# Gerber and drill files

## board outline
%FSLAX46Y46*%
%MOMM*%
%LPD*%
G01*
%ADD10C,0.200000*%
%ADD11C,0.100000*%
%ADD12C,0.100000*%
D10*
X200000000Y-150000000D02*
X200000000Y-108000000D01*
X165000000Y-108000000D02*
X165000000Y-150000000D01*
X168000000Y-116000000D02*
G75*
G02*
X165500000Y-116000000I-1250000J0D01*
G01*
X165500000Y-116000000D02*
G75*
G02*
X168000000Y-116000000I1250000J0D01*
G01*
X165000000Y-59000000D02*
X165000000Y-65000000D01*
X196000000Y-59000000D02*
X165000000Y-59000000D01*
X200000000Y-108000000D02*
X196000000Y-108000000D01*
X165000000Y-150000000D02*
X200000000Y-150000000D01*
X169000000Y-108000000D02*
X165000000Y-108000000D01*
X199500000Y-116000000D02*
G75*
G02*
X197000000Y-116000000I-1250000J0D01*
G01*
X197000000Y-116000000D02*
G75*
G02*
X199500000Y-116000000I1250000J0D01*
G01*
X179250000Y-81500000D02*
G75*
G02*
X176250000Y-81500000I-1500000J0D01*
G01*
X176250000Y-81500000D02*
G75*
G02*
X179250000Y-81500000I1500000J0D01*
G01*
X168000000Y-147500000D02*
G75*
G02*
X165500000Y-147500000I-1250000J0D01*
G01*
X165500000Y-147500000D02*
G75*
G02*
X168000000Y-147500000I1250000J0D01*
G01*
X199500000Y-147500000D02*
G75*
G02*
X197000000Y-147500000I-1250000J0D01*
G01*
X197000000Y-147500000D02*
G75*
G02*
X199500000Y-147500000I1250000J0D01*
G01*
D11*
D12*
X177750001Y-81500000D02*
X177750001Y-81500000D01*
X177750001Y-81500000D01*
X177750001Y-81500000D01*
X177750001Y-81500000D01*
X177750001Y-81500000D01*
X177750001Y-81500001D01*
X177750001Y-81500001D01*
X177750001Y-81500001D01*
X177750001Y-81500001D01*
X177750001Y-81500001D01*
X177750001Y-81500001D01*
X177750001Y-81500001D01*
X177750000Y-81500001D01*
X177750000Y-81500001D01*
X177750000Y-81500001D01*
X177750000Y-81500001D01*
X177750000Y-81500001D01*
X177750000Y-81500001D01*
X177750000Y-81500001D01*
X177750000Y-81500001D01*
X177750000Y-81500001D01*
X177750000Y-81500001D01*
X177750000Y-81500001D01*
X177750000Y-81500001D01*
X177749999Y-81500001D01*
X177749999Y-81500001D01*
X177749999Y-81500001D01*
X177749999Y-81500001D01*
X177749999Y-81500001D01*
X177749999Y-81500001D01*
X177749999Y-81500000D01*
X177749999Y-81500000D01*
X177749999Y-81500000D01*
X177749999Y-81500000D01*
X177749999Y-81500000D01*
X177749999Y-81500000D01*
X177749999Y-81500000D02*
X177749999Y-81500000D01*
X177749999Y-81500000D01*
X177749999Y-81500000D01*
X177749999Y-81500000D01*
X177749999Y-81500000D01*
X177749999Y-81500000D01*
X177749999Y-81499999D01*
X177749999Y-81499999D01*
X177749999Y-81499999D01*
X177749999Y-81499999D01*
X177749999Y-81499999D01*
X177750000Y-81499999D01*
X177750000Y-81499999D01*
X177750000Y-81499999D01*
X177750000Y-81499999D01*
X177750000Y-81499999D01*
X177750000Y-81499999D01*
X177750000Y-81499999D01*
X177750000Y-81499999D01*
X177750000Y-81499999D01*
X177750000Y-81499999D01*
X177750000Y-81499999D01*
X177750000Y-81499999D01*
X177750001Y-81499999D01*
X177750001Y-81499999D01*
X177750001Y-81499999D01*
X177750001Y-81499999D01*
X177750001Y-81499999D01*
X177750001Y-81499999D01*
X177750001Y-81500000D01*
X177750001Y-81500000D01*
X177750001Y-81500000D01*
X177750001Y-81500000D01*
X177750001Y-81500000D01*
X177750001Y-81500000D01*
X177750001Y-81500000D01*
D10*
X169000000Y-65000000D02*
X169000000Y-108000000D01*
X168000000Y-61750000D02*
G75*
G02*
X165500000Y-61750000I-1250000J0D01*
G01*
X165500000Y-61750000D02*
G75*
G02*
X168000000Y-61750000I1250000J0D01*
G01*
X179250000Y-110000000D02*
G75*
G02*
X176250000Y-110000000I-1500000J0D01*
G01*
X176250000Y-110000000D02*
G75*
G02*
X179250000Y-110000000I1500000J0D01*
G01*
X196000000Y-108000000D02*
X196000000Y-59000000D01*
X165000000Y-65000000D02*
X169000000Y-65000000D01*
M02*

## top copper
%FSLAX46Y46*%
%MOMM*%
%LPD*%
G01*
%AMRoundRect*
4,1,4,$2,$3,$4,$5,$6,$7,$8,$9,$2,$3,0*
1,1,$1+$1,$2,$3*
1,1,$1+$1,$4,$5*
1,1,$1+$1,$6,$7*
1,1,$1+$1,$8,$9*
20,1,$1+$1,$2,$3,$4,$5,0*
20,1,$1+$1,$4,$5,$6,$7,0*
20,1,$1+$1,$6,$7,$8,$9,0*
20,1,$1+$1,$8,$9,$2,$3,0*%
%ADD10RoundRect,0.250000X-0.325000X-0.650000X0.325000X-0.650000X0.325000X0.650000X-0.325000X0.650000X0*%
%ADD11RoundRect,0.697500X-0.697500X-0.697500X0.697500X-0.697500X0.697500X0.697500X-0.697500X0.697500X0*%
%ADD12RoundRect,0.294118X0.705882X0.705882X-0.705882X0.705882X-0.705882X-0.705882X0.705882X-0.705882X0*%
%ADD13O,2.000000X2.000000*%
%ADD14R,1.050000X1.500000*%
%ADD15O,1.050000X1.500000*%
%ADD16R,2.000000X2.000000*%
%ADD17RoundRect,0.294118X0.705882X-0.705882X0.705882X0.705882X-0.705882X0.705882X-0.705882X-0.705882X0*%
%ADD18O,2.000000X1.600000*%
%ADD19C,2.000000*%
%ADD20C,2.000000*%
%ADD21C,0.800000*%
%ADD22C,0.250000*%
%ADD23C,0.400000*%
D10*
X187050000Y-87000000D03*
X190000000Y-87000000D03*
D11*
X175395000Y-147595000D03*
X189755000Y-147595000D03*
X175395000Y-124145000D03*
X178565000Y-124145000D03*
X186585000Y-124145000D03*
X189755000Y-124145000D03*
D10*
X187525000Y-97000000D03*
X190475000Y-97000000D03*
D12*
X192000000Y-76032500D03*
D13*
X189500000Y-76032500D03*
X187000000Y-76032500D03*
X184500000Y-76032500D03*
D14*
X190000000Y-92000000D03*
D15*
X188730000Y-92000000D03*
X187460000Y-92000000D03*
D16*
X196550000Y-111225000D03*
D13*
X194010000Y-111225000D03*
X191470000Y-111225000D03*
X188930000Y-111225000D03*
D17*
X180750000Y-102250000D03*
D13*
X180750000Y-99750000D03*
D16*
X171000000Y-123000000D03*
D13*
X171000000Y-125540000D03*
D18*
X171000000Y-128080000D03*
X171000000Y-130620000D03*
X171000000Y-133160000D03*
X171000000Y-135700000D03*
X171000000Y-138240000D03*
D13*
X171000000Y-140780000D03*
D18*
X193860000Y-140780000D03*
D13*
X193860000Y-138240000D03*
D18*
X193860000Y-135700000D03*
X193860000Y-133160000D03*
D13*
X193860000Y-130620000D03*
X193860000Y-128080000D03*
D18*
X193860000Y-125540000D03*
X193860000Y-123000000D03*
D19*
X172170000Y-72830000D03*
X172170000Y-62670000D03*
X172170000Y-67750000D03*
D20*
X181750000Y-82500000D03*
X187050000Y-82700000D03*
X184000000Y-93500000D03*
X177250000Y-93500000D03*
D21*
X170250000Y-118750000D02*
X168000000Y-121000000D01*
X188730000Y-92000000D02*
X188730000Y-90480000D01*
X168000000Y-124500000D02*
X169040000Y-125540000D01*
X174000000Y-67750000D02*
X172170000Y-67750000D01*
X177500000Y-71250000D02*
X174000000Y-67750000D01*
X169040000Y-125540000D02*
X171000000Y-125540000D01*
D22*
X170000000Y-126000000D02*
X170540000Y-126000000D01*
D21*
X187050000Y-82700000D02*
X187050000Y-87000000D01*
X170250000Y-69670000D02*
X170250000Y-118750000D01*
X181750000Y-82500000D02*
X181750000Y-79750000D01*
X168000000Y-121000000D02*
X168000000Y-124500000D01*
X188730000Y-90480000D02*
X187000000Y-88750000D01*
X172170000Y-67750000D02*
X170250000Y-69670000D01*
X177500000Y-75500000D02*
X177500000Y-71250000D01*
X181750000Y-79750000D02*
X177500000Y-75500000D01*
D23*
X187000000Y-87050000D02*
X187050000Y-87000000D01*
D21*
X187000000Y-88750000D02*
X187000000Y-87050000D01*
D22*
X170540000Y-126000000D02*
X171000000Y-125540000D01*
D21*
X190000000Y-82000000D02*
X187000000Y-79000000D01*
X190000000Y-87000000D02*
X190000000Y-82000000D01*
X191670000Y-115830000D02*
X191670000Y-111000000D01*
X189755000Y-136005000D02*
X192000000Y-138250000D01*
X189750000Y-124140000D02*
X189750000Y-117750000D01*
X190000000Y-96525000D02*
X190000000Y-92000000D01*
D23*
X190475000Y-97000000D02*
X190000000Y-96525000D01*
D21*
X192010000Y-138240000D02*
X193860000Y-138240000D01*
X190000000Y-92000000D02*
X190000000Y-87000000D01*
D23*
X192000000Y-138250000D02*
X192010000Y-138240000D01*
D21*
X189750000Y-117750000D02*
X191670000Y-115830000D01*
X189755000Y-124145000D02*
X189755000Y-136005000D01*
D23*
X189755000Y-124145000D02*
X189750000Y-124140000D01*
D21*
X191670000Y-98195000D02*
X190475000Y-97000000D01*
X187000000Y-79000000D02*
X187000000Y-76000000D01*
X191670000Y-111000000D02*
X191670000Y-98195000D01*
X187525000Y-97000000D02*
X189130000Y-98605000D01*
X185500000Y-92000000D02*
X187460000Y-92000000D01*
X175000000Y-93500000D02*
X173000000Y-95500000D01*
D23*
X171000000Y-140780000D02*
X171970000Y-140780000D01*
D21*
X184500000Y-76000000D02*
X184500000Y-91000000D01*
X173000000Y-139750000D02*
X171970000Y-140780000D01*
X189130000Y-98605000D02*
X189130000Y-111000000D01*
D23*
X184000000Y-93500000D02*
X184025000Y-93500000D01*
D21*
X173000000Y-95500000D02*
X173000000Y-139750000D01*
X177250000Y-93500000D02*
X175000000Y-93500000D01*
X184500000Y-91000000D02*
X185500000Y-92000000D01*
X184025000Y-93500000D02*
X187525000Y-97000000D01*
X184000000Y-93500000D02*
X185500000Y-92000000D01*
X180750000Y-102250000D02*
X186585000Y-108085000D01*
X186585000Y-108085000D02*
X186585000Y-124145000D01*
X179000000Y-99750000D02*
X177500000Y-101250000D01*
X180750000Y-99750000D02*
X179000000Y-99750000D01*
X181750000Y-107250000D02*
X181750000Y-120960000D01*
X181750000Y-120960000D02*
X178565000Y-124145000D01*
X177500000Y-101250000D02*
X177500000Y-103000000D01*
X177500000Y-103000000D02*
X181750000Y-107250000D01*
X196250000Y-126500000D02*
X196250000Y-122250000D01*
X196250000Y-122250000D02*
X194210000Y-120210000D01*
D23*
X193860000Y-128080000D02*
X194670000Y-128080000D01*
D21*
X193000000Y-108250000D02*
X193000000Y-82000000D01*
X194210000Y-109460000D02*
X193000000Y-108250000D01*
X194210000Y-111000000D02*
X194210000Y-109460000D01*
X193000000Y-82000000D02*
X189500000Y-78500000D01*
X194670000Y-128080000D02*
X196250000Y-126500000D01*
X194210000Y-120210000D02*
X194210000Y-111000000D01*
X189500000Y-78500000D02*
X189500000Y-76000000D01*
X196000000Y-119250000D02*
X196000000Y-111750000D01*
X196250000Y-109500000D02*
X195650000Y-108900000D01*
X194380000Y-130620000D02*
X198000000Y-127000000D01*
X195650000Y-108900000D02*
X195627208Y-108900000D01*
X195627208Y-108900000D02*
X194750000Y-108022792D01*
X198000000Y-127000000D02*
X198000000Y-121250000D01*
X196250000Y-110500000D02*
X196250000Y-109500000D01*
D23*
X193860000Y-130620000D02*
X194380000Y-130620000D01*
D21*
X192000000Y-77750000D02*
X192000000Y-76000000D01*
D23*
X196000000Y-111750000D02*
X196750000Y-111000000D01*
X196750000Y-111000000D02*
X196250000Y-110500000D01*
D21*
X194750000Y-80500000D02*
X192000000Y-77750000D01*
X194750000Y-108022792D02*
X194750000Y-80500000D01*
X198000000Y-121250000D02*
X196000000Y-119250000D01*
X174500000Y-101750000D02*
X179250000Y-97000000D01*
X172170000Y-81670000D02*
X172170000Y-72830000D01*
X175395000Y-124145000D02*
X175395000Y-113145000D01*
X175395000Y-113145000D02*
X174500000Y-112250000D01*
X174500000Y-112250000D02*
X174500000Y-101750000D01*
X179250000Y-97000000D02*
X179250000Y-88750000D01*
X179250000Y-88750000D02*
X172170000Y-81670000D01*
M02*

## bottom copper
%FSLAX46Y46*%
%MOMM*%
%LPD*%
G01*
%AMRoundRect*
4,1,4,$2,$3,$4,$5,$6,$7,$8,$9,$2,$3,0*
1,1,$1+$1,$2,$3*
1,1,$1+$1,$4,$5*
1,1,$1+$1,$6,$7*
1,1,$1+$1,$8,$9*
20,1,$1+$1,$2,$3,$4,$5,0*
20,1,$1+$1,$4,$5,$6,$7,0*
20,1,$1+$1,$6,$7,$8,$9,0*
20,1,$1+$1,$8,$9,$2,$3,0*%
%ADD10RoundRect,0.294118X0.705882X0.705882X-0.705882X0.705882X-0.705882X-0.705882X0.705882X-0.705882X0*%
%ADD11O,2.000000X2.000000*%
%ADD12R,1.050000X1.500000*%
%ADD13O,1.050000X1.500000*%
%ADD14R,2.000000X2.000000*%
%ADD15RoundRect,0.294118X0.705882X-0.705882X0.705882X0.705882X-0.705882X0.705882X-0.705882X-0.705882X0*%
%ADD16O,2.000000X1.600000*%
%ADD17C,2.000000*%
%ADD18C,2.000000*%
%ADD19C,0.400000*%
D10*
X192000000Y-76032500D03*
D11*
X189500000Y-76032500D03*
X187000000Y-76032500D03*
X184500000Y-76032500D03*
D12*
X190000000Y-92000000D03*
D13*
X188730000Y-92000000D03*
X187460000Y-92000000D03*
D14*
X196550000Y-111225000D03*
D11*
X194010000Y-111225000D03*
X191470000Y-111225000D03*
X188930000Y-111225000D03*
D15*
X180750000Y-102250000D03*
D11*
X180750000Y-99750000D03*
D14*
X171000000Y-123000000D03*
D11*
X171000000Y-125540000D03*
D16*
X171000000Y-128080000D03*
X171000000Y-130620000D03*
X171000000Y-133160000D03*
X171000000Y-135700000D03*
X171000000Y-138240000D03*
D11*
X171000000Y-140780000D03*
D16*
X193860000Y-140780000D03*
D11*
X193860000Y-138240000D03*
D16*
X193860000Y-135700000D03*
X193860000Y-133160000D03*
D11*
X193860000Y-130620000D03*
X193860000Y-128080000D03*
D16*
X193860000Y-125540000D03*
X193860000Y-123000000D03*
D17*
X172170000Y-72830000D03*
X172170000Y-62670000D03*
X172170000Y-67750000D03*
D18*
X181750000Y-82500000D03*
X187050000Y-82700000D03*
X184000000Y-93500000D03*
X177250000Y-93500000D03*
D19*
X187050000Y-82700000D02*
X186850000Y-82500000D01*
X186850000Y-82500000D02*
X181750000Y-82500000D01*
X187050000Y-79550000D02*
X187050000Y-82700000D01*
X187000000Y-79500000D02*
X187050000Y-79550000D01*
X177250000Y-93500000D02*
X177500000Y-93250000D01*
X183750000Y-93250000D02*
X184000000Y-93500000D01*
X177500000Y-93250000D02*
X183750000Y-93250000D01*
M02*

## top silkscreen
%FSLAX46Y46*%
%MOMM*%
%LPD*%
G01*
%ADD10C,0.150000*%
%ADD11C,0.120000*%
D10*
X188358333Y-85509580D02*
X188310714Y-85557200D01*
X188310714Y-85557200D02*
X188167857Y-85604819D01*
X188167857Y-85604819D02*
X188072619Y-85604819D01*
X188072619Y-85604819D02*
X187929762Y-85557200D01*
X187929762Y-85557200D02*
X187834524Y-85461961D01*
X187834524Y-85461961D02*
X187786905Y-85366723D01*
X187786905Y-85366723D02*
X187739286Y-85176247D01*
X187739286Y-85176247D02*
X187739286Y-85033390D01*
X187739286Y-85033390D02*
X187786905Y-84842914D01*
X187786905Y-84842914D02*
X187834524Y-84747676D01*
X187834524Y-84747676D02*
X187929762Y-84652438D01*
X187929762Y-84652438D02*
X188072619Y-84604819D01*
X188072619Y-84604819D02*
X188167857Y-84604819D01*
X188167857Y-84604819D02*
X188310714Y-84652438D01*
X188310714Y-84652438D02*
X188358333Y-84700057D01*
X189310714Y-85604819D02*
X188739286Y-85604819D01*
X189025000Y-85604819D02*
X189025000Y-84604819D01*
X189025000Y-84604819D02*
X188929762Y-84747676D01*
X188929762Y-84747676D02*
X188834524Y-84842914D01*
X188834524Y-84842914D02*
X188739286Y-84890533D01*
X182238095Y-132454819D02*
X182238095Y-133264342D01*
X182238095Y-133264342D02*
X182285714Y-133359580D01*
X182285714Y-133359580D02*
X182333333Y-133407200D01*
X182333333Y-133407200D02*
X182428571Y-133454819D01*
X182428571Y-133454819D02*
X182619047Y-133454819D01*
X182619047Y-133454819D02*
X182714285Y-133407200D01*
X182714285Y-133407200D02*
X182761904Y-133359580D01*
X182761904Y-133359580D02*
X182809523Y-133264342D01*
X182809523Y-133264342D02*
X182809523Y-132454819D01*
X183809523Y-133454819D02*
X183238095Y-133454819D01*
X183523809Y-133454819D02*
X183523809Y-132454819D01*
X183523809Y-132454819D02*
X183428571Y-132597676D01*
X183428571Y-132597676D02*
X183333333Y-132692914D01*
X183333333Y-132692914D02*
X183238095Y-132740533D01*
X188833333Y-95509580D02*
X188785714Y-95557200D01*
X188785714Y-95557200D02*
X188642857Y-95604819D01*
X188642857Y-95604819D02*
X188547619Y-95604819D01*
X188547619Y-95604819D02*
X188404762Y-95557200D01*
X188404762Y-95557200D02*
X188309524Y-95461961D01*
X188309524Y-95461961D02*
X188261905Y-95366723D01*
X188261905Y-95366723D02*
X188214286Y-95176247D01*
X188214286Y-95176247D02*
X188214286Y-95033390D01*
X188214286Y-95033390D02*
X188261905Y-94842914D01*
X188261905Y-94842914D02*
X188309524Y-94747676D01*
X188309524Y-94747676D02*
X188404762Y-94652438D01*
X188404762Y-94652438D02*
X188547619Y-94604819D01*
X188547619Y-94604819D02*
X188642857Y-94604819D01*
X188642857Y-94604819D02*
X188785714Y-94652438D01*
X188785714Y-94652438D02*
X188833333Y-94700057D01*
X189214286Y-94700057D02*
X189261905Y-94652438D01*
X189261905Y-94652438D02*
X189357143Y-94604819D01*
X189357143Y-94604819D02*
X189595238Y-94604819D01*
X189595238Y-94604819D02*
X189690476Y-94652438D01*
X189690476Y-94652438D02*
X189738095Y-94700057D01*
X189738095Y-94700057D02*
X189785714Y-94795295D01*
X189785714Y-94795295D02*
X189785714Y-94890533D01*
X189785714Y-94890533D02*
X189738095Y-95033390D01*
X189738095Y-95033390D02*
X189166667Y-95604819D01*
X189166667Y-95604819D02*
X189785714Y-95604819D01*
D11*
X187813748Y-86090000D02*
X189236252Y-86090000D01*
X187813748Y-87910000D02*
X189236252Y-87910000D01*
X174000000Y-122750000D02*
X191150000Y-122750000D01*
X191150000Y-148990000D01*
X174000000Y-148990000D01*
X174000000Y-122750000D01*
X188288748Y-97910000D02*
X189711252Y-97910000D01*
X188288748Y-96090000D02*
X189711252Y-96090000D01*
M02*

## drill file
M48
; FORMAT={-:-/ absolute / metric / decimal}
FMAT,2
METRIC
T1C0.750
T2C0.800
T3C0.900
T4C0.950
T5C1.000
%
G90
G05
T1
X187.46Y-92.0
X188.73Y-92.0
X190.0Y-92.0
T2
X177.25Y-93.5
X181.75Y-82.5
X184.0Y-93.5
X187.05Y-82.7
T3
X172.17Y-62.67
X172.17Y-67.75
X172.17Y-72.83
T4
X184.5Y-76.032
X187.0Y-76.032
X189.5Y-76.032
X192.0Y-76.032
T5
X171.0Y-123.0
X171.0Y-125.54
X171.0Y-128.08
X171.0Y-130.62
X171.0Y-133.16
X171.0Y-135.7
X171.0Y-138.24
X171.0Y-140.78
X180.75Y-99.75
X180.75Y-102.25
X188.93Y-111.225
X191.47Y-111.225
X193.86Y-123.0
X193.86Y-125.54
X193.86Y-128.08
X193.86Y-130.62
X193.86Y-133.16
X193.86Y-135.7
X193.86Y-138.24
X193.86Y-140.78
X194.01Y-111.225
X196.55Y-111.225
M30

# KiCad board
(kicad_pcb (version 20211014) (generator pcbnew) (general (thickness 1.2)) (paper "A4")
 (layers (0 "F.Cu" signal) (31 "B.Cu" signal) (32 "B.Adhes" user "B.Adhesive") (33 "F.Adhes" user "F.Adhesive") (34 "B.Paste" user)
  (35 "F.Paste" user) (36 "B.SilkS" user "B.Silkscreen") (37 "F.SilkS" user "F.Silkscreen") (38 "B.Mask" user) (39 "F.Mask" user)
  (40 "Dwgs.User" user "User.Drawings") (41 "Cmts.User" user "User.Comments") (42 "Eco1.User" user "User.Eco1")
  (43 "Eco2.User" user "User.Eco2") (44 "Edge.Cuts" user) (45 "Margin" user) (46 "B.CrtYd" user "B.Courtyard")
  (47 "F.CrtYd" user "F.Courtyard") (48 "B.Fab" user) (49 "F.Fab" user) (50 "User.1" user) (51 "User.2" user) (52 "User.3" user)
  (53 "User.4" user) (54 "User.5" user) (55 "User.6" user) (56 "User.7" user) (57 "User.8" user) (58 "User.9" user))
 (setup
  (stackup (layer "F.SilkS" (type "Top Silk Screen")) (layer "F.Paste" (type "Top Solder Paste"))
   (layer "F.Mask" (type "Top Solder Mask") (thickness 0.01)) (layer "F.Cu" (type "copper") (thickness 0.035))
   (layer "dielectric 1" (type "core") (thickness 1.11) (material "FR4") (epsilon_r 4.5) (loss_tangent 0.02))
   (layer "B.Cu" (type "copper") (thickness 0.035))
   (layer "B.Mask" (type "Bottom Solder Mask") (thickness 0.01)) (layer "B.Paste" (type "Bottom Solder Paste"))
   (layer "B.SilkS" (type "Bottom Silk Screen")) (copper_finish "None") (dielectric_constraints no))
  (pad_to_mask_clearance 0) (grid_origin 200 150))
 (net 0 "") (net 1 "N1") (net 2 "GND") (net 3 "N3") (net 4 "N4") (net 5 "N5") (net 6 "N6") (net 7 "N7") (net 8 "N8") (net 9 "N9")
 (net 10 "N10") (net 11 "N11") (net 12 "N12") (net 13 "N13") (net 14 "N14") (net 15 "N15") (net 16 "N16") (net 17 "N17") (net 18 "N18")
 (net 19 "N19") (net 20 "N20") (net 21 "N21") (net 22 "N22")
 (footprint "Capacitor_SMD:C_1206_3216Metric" (layer "F.Cu") (at 188.525 87)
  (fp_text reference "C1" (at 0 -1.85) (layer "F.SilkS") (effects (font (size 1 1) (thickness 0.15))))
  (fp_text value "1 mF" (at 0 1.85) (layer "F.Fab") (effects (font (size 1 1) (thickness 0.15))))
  (fp_line (start -0.711252 -0.91) (end 0.711252 -0.91) (layer "F.SilkS") (width 0.12))
  (fp_line (start -0.711252 0.91) (end 0.711252 0.91) (layer "F.SilkS") (width 0.12))
  (pad "1" smd roundrect (at -1.475 0) (size 1.15 1.8) (layers "F.Cu" "F.Paste" "F.Mask") (roundrect_rratio 0.217391) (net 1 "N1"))
  (pad "2" smd roundrect (at 1.475 0) (size 1.15 1.8) (layers "F.Cu" "F.Paste" "F.Mask") (roundrect_rratio 0.217391) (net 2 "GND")))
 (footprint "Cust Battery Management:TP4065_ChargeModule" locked (layer "F.Cu") (at 174 122.75)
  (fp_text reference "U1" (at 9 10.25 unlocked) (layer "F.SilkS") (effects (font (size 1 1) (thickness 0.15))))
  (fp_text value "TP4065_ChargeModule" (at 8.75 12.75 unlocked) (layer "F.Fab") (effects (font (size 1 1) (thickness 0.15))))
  (fp_rect (start 0 0) (end 17.15 26.24) (layer "F.SilkS") (width 0.12) (fill none))
  (pad "1" smd roundrect locked (at 1.395 24.845) (size 2.79 2.79) (layers "F.Cu" "F.Paste" "F.Mask") (roundrect_rratio 0.25) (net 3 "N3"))
  (pad "2" smd roundrect locked (at 15.755 24.845) (size 2.79 2.79) (layers "F.Cu" "F.Paste" "F.Mask") (roundrect_rratio 0.25) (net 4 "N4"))
  (pad "3" smd roundrect locked (at 1.395 1.395) (size 2.79 2.79) (layers "F.Cu" "F.Paste" "F.Mask") (roundrect_rratio 0.25) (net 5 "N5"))
  (pad "4" smd roundrect locked (at 4.565 1.395) (size 2.79 2.79) (layers "F.Cu" "F.Paste" "F.Mask") (roundrect_rratio 0.25) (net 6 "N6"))
  (pad "5" smd roundrect locked (at 12.585 1.395) (size 2.79 2.79) (layers "F.Cu" "F.Paste" "F.Mask") (roundrect_rratio 0.25) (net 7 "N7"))
  (pad "6" smd roundrect locked (at 15.755 1.395) (size 2.79 2.79) (layers "F.Cu" "F.Paste" "F.Mask") (roundrect_rratio 0.25) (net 2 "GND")))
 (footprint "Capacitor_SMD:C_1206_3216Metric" (layer "F.Cu") (at 189 97)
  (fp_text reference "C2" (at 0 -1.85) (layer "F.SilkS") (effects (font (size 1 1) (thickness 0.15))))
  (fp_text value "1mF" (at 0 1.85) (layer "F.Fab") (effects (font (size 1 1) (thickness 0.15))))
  (fp_line (start -0.711252 0.91) (end 0.711252 0.91) (layer "F.SilkS") (width 0.12))
  (fp_line (start -0.711252 -0.91) (end 0.711252 -0.91) (layer "F.SilkS") (width 0.12))
  (pad "1" smd roundrect (at -1.475 0) (size 1.15 1.8) (layers "F.Cu" "F.Paste" "F.Mask") (roundrect_rratio 0.217391) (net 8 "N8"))
  (pad "2" smd roundrect (at 1.475 0) (size 1.15 1.8) (layers "F.Cu" "F.Paste" "F.Mask") (roundrect_rratio 0.217391) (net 2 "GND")))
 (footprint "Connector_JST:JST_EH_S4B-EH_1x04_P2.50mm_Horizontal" (layer "B.Cu") (at 192 76.0325 180)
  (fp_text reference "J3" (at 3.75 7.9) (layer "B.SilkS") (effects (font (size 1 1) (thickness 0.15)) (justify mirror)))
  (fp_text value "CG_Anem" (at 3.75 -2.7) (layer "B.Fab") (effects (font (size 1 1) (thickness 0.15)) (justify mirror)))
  (pad "1" thru_hole roundrect (at 0 0 180) (size 2 2) (drill 0.95) (layers *.Cu *.Mask) (roundrect_rratio 0.147059) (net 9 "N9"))
  (pad "2" thru_hole oval (at 2.5 0 180) (size 2 2) (drill 0.95) (layers *.Cu *.Mask) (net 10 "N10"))
  (pad "3" thru_hole oval (at 5 0 180) (size 2 2) (drill 0.95) (layers *.Cu *.Mask) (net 2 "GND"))
  (pad "4" thru_hole oval (at 7.5 0 180) (size 2 2) (drill 0.95) (layers *.Cu *.Mask) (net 8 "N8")))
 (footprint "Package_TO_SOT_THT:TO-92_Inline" (layer "B.Cu") (at 190 92 180)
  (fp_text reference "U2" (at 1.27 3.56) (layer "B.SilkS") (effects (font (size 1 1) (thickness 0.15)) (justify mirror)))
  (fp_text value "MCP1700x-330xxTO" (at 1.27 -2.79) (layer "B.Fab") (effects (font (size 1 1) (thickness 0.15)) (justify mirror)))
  (pad "1" thru_hole rect (at 0 0 180) (size 1.05 1.5) (drill 0.75) (layers *.Cu *.Mask) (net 2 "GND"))
  (pad "2" thru_hole oval (at 1.27 0 180) (size 1.05 1.5) (drill 0.75) (layers *.Cu *.Mask) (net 1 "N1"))
  (pad "3" thru_hole oval (at 2.54 0 180) (size 1.05 1.5) (drill 0.75) (layers *.Cu *.Mask) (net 8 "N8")))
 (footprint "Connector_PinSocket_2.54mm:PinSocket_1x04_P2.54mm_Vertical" (layer "B.Cu") (at 196.55 111.225 90)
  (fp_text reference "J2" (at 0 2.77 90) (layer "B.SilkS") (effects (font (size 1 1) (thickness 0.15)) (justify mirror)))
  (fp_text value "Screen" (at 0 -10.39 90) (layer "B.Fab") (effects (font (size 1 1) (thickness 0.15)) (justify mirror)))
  (pad "1" thru_hole rect locked (at 0 0 90) (size 2 2) (drill 1) (layers *.Cu *.Mask) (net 9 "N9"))
  (pad "2" thru_hole oval locked (at 0 -2.54 90) (size 2 2) (drill 1) (layers *.Cu *.Mask) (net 10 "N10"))
  (pad "3" thru_hole oval locked (at 0 -5.08 90) (size 2 2) (drill 1) (layers *.Cu *.Mask) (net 2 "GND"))
  (pad "4" thru_hole oval locked (at 0 -7.62 90) (size 2 2) (drill 1) (layers *.Cu *.Mask) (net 8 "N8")))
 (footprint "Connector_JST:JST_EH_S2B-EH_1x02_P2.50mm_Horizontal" (layer "B.Cu") (at 180.75 102.25 90)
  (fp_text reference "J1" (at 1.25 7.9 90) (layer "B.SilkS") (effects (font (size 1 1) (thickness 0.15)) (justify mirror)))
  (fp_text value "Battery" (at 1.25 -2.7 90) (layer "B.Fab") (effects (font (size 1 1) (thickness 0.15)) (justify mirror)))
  (pad "1" thru_hole roundrect (at 0 0 90) (size 2 2) (drill 1) (layers *.Cu *.Mask) (roundrect_rratio 0.147059) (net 7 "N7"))
  (pad "2" thru_hole oval (at 2.5 0 90) (size 2 2) (drill 1) (layers *.Cu *.Mask) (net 6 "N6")))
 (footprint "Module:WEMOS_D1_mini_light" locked (layer "B.Cu") (at 193 123 180)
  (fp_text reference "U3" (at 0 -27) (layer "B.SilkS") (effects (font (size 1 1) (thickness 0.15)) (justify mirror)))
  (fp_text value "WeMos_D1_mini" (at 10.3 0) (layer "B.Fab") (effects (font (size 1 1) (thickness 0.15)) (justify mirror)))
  (pad "1" thru_hole rect locked (at 22 0 180) (size 2 2) (drill 1) (layers *.Cu *.Mask) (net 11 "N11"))
  (pad "2" thru_hole oval locked (at 22 -2.54 180) (size 2 2) (drill 1) (layers *.Cu *.Mask) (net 1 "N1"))
  (pad "3" thru_hole oval locked (at 22 -5.08 180) (size 2 1.6) (drill 1) (layers *.Cu *.Mask) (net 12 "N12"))
  (pad "4" thru_hole oval locked (at 22 -7.62 180) (size 2 1.6) (drill 1) (layers *.Cu *.Mask) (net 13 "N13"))
  (pad "5" thru_hole oval locked (at 22 -10.16 180) (size 2 1.6) (drill 1) (layers *.Cu *.Mask) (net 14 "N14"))
  (pad "6" thru_hole oval locked (at 22 -12.7 180) (size 2 1.6) (drill 1) (layers *.Cu *.Mask) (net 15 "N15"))
  (pad "7" thru_hole oval locked (at 22 -15.24 180) (size 2 1.6) (drill 1) (layers *.Cu *.Mask) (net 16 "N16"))
  (pad "8" thru_hole oval locked (at 22 -17.78 180) (size 2 2) (drill 1) (layers *.Cu *.Mask) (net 8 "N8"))
  (pad "9" thru_hole oval locked (at -0.86 -17.78 180) (size 2 1.6) (drill 1) (layers *.Cu *.Mask) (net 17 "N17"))
  (pad "10" thru_hole oval locked (at -0.86 -15.24 180) (size 2 2) (drill 1) (layers *.Cu *.Mask) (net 2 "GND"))
  (pad "11" thru_hole oval locked (at -0.86 -12.7 180) (size 2 1.6) (drill 1) (layers *.Cu *.Mask) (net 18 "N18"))
  (pad "12" thru_hole oval locked (at -0.86 -10.16 180) (size 2 1.6) (drill 1) (layers *.Cu *.Mask) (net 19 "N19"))
  (pad "13" thru_hole oval locked (at -0.86 -7.62 180) (size 2 2) (drill 1) (layers *.Cu *.Mask) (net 9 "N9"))
  (pad "14" thru_hole oval locked (at -0.86 -5.08 180) (size 2 2) (drill 1) (layers *.Cu *.Mask) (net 10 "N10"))
  (pad "15" thru_hole oval locked (at -0.86 -2.54 180) (size 2 1.6) (drill 1) (layers *.Cu *.Mask) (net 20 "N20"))
  (pad "16" thru_hole oval locked (at -0.86 0 180) (size 2 1.6) (drill 1) (layers *.Cu *.Mask) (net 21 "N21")))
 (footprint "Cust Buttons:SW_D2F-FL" (layer "B.Cu") (at 172.17 67.75 90)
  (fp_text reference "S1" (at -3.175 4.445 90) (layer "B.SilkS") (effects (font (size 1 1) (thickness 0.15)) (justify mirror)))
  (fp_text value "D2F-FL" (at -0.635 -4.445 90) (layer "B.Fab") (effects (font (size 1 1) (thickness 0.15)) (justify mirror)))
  (pad "COM" thru_hole circle locked (at -5.08 0 90) (size 2 2) (drill 0.9) (layers *.Cu *.Mask) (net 5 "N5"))
  (pad "NC" thru_hole circle locked (at 5.08 0 90) (size 2 2) (drill 0.9) (layers *.Cu *.Mask) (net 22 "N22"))
  (pad "NO" thru_hole circle locked (at 0 0 90) (size 2 2) (drill 0.9) (layers *.Cu *.Mask) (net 1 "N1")))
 (gr_line locked (start 200 150) (end 200 108) (layer "Edge.Cuts") (width 0.2))
 (gr_line locked (start 165 108) (end 165 150) (layer "Edge.Cuts") (width 0.2))
 (gr_circle locked (center 166.75 116) (end 168 116) (layer "Edge.Cuts") (width 0.2) (fill none))
 (gr_line locked (start 165 59) (end 165 65) (layer "Edge.Cuts") (width 0.2))
 (gr_line locked (start 196 59) (end 165 59) (layer "Edge.Cuts") (width 0.2))
 (gr_line (start 200 108) (end 196 108) (layer "Edge.Cuts") (width 0.2))
 (gr_line locked (start 165 150) (end 200 150) (layer "Edge.Cuts") (width 0.2))
 (gr_line locked (start 169 108) (end 165 108) (layer "Edge.Cuts") (width 0.2))
 (gr_circle locked (center 198.25 116) (end 199.5 116) (layer "Edge.Cuts") (width 0.2) (fill none))
 (gr_circle locked (center 177.75 81.5) (end 179.25 81.5) (layer "Edge.Cuts") (width 0.2) (fill none))
 (gr_circle locked (center 166.75 147.5) (end 168 147.5) (layer "Edge.Cuts") (width 0.2) (fill none))
 (gr_circle locked (center 198.25 147.5) (end 199.5 147.5) (layer "Edge.Cuts") (width 0.2) (fill none))
 (gr_circle (center 177.75 81.5) (end 177.75 81.5) (layer "Edge.Cuts") (width 0.1) (fill none))
 (gr_line locked (start 169 65) (end 169 108) (layer "Edge.Cuts") (width 0.2))
 (gr_circle locked (center 166.75 61.75) (end 168 61.75) (layer "Edge.Cuts") (width 0.2) (fill none))
 (gr_circle locked (center 177.75 110) (end 179.25 110) (layer "Edge.Cuts") (width 0.2) (fill none))
 (gr_line locked (start 196 108) (end 196 59) (layer "Edge.Cuts") (width 0.2))
 (gr_line locked (start 165 65) (end 169 65) (layer "Edge.Cuts") (width 0.2))
 (segment (start 170.25 118.75) (end 168 121) (width 0.8) (layer "F.Cu") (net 1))
 (segment (start 188.73 92) (end 188.73 90.48) (width 0.8) (layer "F.Cu") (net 1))
 (segment (start 168 124.5) (end 169.04 125.54) (width 0.8) (layer "F.Cu") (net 1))
 (segment (start 174 67.75) (end 172.17 67.75) (width 0.8) (layer "F.Cu") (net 1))
 (segment (start 177.5 71.25) (end 174 67.75) (width 0.8) (layer "F.Cu") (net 1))
 (segment (start 169.04 125.54) (end 171 125.54) (width 0.8) (layer "F.Cu") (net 1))
 (segment (start 170 126) (end 170.54 126) (width 0.25) (layer "F.Cu") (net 1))
 (segment (start 187.05 82.7) (end 187.05 87) (width 0.8) (layer "F.Cu") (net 1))
 (segment (start 170.25 69.67) (end 170.25 118.75) (width 0.8) (layer "F.Cu") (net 1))
 (segment (start 181.75 82.5) (end 181.75 79.75) (width 0.8) (layer "F.Cu") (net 1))
 (segment (start 168 121) (end 168 124.5) (width 0.8) (layer "F.Cu") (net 1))
 (segment (start 188.73 90.48) (end 187 88.75) (width 0.8) (layer "F.Cu") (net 1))
 (segment (start 172.17 67.75) (end 170.25 69.67) (width 0.8) (layer "F.Cu") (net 1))
 (segment (start 177.5 75.5) (end 177.5 71.25) (width 0.8) (layer "F.Cu") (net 1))
 (segment (start 181.75 79.75) (end 177.5 75.5) (width 0.8) (layer "F.Cu") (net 1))
 (segment (start 187 87.05) (end 187.05 87) (width 0.4) (layer "F.Cu") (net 1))
 (segment (start 187 88.75) (end 187 87.05) (width 0.8) (layer "F.Cu") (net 1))
 (segment (start 170.54 126) (end 171 125.54) (width 0.25) (layer "F.Cu") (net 1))
 (via (at 181.75 82.5) (size 2) (drill 0.8) (layers "F.Cu" "B.Cu") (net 1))
 (via (at 187.05 82.7) (size 2) (drill 0.8) (layers "F.Cu" "B.Cu") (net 1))
 (segment (start 187.05 82.7) (end 186.85 82.5) (width 0.4) (layer "B.Cu") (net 1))
 (segment (start 186.85 82.5) (end 181.75 82.5) (width 0.4) (layer "B.Cu") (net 1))
 (segment (start 187.05 79.55) (end 187.05 82.7) (width 0.4) (layer "B.Cu") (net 1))
 (segment (start 187 79.5) (end 187.05 79.55) (width 0.4) (layer "B.Cu") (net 1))
 (segment (start 190 82) (end 187 79) (width 0.8) (layer "F.Cu") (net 2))
 (segment (start 190 87) (end 190 82) (width 0.8) (layer "F.Cu") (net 2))
 (segment (start 191.67 115.83) (end 191.67 111) (width 0.8) (layer "F.Cu") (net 2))
 (segment (start 189.755 136.005) (end 192 138.25) (width 0.8) (layer "F.Cu") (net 2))
 (segment (start 189.75 124.14) (end 189.75 117.75) (width 0.8) (layer "F.Cu") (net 2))
 (segment (start 190 96.525) (end 190 92) (width 0.8) (layer "F.Cu") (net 2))
 (segment (start 190.475 97) (end 190 96.525) (width 0.4) (layer "F.Cu") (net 2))
 (segment (start 192.01 138.24) (end 193.86 138.24) (width 0.8) (layer "F.Cu") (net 2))
 (segment (start 190 92) (end 190 87) (width 0.8) (layer "F.Cu") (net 2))
 (segment (start 192 138.25) (end 192.01 138.24) (width 0.4) (layer "F.Cu") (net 2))
 (segment (start 189.75 117.75) (end 191.67 115.83) (width 0.8) (layer "F.Cu") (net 2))
 (segment (start 189.755 124.145) (end 189.755 136.005) (width 0.8) (layer "F.Cu") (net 2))
 (segment (start 189.755 124.145) (end 189.75 124.14) (width 0.4) (layer "F.Cu") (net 2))
 (segment (start 191.67 98.195) (end 190.475 97) (width 0.8) (layer "F.Cu") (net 2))
 (segment (start 187 79) (end 187 76) (width 0.8) (layer "F.Cu") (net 2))
 (segment (start 191.67 111) (end 191.67 98.195) (width 0.8) (layer "F.Cu") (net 2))
 (segment (start 187.525 97) (end 189.13 98.605) (width 0.8) (layer "F.Cu") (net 8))
 (segment (start 185.5 92) (end 187.46 92) (width 0.8) (layer "F.Cu") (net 8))
 (segment (start 175 93.5) (end 173 95.5) (width 0.8) (layer "F.Cu") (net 8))
 (segment (start 171 140.78) (end 171.97 140.78) (width 0.4) (layer "F.Cu") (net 8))
 (segment (start 184.5 76) (end 184.5 91) (width 0.8) (layer "F.Cu") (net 8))
 (segment (start 173 139.75) (end 171.97 140.78) (width 0.8) (layer "F.Cu") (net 8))
 (segment (start 189.13 98.605) (end 189.13 111) (width 0.8) (layer "F.Cu") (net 8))
 (segment (start 184 93.5) (end 184.025 93.5) (width 0.4) (layer "F.Cu") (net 8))
 (segment (start 173 95.5) (end 173 139.75) (width 0.8) (layer "F.Cu") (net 8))
 (segment (start 177.25 93.5) (end 175 93.5) (width 0.8) (layer "F.Cu") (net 8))
 (segment (start 184.5 91) (end 185.5 92) (width 0.8) (layer "F.Cu") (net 8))
 (segment (start 184.025 93.5) (end 187.525 97) (width 0.8) (layer "F.Cu") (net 8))
 (segment (start 184 93.5) (end 185.5 92) (width 0.8) (layer "F.Cu") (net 8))
 (via (at 184 93.5) (size 2) (drill 0.8) (layers "F.Cu" "B.Cu") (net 8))
 (via (at 177.25 93.5) (size 2) (drill 0.8) (layers "F.Cu" "B.Cu") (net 8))
 (segment (start 177.25 93.5) (end 177.5 93.25) (width 0.4) (layer "B.Cu") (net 8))
 (segment (start 183.75 93.25) (end 184 93.5) (width 0.4) (layer "B.Cu") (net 8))
 (segment (start 177.5 93.25) (end 183.75 93.25) (width 0.4) (layer "B.Cu") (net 8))
 (segment (start 180.75 102.25) (end 186.585 108.085) (width 0.8) (layer "F.Cu") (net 7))
 (segment (start 186.585 108.085) (end 186.585 124.145) (width 0.8) (layer "F.Cu") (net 7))
 (segment (start 179 99.75) (end 177.5 101.25) (width 0.8) (layer "F.Cu") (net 6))
 (segment (start 180.75 99.75) (end 179 99.75) (width 0.8) (layer "F.Cu") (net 6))
 (segment (start 181.75 107.25) (end 181.75 120.96) (width 0.8) (layer "F.Cu") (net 6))
 (segment (start 181.75 120.96) (end 178.565 124.145) (width 0.8) (layer "F.Cu") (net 6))
 (segment (start 177.5 101.25) (end 177.5 103) (width 0.8) (layer "F.Cu") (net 6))
 (segment (start 177.5 103) (end 181.75 107.25) (width 0.8) (layer "F.Cu") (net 6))
 (segment (start 196.25 126.5) (end 196.25 122.25) (width 0.8) (layer "F.Cu") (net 10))
 (segment (start 196.25 122.25) (end 194.21 120.21) (width 0.8) (layer "F.Cu") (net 10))
 (segment (start 193.86 128.08) (end 194.67 128.08) (width 0.4) (layer "F.Cu") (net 10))
 (segment (start 193 108.25) (end 193 82) (width 0.8) (layer "F.Cu") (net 10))
 (segment (start 194.21 109.46) (end 193 108.25) (width 0.8) (layer "F.Cu") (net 10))
 (segment (start 194.21 111) (end 194.21 109.46) (width 0.8) (layer "F.Cu") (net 10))
 (segment (start 193 82) (end 189.5 78.5) (width 0.8) (layer "F.Cu") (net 10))
 (segment (start 194.67 128.08) (end 196.25 126.5) (width 0.8) (layer "F.Cu") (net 10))
 (segment (start 194.21 120.21) (end 194.21 111) (width 0.8) (layer "F.Cu") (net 10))
 (segment (start 189.5 78.5) (end 189.5 76) (width 0.8) (layer "F.Cu") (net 10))
 (segment (start 196 119.25) (end 196 111.75) (width 0.8) (layer "F.Cu") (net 9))
 (segment (start 196.25 109.5) (end 195.65 108.9) (width 0.8) (layer "F.Cu") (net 9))
 (segment (start 194.38 130.62) (end 198 127) (width 0.8) (layer "F.Cu") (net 9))
 (segment (start 195.65 108.9) (end 195.627208 108.9) (width 0.8) (layer "F.Cu") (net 9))
 (segment (start 195.627208 108.9) (end 194.75 108.022792) (width 0.8) (layer "F.Cu") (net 9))
 (segment (start 198 127) (end 198 121.25) (width 0.8) (layer "F.Cu") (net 9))
 (segment (start 196.25 110.5) (end 196.25 109.5) (width 0.8) (layer "F.Cu") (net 9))
 (segment (start 193.86 130.62) (end 194.38 130.62) (width 0.4) (layer "F.Cu") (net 9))
 (segment (start 192 77.75) (end 192 76) (width 0.8) (layer "F.Cu") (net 9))
 (segment (start 196 111.75) (end 196.75 111) (width 0.4) (layer "F.Cu") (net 9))
 (segment (start 196.75 111) (end 196.25 110.5) (width 0.4) (layer "F.Cu") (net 9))
 (segment (start 194.75 80.5) (end 192 77.75) (width 0.8) (layer "F.Cu") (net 9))
 (segment (start 194.75 108.022792) (end 194.75 80.5) (width 0.8) (layer "F.Cu") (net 9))
 (segment (start 198 121.25) (end 196 119.25) (width 0.8) (layer "F.Cu") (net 9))
 (segment (start 174.5 101.75) (end 179.25 97) (width 0.8) (layer "F.Cu") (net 5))
 (segment (start 172.17 81.67) (end 172.17 72.83) (width 0.8) (layer "F.Cu") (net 5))
 (segment (start 175.395 124.145) (end 175.395 113.145) (width 0.8) (layer "F.Cu") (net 5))
 (segment (start 175.395 113.145) (end 174.5 112.25) (width 0.8) (layer "F.Cu") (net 5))
 (segment (start 174.5 112.25) (end 174.5 101.75) (width 0.8) (layer "F.Cu") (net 5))
 (segment (start 179.25 97) (end 179.25 88.75) (width 0.8) (layer "F.Cu") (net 5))
 (segment (start 179.25 88.75) (end 172.17 81.67) (width 0.8) (layer "F.Cu") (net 5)))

